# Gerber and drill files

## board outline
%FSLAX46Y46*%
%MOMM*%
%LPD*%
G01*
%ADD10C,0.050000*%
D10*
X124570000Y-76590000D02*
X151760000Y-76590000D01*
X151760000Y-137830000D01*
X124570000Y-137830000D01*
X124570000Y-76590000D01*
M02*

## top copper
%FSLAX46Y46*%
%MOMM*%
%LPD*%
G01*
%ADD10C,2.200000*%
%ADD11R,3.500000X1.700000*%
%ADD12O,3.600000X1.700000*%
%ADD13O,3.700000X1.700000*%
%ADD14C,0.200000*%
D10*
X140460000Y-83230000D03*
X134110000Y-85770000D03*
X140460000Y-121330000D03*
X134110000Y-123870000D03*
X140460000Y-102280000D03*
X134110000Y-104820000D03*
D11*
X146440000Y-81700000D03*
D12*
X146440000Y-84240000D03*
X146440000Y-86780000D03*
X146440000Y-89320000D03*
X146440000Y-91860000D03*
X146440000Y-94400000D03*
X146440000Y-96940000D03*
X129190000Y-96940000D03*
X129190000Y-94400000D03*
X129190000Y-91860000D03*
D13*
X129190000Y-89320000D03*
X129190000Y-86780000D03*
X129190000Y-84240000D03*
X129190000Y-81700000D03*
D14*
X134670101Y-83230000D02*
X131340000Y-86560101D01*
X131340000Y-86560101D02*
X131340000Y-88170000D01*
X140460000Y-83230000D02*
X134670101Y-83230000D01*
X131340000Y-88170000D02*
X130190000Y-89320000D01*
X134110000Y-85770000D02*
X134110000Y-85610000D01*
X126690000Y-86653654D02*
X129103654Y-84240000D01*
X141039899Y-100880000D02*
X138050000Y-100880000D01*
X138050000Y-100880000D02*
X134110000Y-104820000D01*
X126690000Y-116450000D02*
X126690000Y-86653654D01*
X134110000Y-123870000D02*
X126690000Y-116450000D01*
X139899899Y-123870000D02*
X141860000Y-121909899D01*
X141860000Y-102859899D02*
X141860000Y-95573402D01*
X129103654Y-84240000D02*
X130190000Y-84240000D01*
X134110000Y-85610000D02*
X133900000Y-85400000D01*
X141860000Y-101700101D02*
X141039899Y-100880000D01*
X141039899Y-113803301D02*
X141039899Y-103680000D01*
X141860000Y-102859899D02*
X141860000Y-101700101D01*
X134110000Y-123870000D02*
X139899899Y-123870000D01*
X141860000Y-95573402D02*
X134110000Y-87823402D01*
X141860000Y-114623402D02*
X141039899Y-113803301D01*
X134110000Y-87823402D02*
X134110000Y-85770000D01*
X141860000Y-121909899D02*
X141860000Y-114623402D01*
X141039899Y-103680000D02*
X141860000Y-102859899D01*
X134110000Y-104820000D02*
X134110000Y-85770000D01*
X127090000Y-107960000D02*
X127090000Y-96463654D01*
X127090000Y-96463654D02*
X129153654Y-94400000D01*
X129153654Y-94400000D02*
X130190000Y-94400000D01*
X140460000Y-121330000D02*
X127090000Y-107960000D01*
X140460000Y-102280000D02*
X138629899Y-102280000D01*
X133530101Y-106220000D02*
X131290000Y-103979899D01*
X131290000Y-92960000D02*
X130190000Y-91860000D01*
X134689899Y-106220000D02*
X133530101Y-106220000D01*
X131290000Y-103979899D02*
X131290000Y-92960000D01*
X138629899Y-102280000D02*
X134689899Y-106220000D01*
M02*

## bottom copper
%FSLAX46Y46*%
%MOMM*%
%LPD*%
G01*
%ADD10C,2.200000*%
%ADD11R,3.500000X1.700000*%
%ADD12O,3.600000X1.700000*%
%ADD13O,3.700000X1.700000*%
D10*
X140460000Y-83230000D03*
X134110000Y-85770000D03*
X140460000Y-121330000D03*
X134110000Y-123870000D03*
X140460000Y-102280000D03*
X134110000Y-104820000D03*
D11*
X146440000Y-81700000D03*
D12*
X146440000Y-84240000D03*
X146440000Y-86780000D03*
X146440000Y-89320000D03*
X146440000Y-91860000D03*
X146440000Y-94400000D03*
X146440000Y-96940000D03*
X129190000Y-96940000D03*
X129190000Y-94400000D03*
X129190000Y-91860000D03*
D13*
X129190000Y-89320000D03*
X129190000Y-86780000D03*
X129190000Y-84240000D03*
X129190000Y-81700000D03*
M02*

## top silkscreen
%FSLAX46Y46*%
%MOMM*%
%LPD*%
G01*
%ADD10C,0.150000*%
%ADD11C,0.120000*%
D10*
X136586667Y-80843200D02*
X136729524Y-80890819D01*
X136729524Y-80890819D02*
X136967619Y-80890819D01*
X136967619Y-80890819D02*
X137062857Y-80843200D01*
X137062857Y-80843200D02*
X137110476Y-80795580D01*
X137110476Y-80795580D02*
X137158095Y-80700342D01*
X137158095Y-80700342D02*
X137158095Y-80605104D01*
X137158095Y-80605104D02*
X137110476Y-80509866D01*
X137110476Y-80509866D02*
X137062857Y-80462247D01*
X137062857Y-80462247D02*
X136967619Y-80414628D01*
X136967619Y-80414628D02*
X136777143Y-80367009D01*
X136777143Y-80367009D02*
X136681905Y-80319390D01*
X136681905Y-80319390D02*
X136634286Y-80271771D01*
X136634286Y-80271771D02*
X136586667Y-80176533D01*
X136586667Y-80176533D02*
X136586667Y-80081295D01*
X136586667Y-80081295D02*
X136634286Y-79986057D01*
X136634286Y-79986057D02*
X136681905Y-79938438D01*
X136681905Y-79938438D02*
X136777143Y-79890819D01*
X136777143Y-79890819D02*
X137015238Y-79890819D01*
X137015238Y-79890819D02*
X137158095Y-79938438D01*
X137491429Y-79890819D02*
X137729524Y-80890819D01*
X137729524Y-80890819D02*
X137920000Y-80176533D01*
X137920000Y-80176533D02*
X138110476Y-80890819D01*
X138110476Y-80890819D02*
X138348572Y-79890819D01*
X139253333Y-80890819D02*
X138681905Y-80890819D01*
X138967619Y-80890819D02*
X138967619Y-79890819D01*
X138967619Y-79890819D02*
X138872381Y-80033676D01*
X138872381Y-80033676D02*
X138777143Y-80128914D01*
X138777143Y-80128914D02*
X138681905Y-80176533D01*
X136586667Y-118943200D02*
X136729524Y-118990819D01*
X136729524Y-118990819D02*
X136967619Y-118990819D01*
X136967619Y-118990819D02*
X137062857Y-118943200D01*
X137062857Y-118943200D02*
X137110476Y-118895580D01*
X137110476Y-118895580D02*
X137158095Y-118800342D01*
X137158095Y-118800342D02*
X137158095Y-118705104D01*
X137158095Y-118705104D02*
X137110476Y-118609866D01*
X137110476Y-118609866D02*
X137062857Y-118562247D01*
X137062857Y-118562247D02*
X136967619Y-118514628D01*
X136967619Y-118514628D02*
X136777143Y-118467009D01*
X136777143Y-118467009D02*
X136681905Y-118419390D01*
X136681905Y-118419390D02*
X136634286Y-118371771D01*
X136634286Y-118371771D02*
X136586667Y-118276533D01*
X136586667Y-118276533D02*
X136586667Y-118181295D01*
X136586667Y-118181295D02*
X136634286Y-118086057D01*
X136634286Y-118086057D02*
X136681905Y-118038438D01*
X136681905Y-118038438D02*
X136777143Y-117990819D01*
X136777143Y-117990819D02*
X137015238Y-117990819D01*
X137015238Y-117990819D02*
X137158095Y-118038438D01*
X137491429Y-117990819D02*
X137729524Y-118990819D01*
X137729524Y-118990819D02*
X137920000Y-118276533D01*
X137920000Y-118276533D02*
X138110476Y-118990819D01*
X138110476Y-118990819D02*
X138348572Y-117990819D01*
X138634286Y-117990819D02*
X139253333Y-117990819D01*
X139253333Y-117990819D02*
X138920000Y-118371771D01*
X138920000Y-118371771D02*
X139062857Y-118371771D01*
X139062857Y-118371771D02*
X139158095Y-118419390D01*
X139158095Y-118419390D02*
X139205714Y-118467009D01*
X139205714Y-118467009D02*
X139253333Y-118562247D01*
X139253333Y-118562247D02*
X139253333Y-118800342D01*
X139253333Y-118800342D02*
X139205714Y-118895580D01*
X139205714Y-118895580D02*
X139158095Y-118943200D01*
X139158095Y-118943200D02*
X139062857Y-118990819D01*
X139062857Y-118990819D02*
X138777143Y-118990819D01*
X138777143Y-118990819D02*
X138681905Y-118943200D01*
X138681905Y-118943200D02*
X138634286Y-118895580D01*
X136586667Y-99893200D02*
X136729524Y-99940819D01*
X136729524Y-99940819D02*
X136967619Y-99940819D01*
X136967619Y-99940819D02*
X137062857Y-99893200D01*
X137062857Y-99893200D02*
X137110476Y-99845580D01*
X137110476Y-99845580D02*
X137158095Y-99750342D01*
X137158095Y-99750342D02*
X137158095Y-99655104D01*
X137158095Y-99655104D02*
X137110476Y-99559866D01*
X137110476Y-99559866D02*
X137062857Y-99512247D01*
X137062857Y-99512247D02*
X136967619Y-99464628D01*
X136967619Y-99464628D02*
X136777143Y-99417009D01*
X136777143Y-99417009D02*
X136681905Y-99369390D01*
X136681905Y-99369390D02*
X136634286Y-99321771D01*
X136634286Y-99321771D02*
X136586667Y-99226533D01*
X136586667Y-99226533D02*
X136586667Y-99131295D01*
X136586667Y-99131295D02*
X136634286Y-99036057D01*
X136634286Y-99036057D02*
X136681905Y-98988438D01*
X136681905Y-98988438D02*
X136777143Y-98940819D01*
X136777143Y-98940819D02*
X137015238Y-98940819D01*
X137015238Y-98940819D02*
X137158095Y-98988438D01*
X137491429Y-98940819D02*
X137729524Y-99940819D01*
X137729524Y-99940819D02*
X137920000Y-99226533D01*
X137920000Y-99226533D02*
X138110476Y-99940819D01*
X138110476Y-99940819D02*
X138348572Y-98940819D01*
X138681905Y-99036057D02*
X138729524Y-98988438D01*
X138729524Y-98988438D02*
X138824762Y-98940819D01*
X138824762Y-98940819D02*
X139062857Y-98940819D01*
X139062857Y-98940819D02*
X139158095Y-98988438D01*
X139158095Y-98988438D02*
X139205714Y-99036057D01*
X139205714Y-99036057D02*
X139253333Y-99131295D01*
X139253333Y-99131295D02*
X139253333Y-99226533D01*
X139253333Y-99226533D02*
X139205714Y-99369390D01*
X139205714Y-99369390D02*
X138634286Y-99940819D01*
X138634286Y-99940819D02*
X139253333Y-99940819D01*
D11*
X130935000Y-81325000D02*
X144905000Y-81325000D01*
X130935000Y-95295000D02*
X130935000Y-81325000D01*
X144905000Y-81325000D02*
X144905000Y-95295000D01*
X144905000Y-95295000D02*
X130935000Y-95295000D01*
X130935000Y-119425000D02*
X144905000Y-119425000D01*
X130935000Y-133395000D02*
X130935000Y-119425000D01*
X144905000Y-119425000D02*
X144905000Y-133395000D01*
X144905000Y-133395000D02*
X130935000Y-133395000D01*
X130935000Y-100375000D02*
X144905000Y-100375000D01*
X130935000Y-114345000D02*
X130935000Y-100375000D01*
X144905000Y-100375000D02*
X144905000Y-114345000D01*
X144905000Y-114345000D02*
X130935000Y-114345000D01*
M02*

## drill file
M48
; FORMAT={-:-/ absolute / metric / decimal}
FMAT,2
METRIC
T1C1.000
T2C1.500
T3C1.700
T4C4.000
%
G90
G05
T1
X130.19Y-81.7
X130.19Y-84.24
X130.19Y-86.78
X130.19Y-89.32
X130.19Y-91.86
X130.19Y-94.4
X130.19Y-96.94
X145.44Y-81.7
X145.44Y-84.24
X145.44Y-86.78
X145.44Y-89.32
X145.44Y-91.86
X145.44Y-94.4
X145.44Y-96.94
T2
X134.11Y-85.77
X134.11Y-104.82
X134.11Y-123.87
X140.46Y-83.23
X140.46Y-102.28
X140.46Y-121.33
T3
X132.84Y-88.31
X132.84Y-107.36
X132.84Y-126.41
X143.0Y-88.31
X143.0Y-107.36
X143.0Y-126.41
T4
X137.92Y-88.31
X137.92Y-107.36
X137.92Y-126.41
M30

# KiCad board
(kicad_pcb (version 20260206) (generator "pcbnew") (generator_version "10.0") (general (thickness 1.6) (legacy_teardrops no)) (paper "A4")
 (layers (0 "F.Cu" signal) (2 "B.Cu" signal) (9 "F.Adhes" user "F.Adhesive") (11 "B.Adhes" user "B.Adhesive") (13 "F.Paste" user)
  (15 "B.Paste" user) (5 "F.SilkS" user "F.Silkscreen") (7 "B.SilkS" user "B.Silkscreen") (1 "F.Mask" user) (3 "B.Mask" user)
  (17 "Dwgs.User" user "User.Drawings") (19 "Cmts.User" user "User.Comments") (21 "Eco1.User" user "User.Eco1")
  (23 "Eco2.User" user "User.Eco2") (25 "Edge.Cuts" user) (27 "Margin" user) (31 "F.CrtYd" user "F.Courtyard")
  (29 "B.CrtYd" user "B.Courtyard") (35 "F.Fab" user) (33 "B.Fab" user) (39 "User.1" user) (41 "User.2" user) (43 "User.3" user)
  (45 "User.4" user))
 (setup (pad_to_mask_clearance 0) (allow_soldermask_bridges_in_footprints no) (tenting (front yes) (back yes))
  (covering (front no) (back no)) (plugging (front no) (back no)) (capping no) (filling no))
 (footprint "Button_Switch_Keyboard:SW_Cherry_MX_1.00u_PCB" (layer "F.Cu") (at 140.46 83.23)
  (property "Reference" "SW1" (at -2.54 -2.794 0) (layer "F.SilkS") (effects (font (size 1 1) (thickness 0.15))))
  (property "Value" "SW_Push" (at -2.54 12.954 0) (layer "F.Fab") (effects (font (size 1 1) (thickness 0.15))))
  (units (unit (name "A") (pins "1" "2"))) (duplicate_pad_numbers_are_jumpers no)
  (fp_line (start -9.525 -1.905) (end 4.445 -1.905) (stroke (width 0.12) (type solid)) (layer "F.SilkS"))
  (fp_line (start -9.525 12.065) (end -9.525 -1.905) (stroke (width 0.12) (type solid)) (layer "F.SilkS"))
  (fp_line (start 4.445 -1.905) (end 4.445 12.065) (stroke (width 0.12) (type solid)) (layer "F.SilkS"))
  (fp_line (start 4.445 12.065) (end -9.525 12.065) (stroke (width 0.12) (type solid)) (layer "F.SilkS"))
  (pad "" np_thru_hole circle (at -7.62 5.08) (size 1.7 1.7) (drill 1.7) (layers "*.Cu" "*.Mask"))
  (pad "" np_thru_hole circle (at -2.54 5.08) (size 4 4) (drill 4) (layers "*.Cu" "*.Mask"))
  (pad "" np_thru_hole circle (at 2.54 5.08) (size 1.7 1.7) (drill 1.7) (layers "*.Cu" "*.Mask"))
  (pad "1" thru_hole circle (at 0 0) (size 2.2 2.2) (drill 1.5) (layers "*.Cu" "*.Mask") (remove_unused_layers no)
   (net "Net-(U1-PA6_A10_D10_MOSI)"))
  (pad "2" thru_hole circle (at -6.35 2.54) (size 2.2 2.2) (drill 1.5) (layers "*.Cu" "*.Mask") (remove_unused_layers no) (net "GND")))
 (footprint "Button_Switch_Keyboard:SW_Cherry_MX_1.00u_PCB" (layer "F.Cu") (at 140.46 121.33)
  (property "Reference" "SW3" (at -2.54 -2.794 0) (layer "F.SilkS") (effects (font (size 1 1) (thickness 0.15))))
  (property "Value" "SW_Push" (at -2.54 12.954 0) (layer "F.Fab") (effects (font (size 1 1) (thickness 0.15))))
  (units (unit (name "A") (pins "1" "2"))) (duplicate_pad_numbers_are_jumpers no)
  (fp_line (start -9.525 -1.905) (end 4.445 -1.905) (stroke (width 0.12) (type solid)) (layer "F.SilkS"))
  (fp_line (start -9.525 12.065) (end -9.525 -1.905) (stroke (width 0.12) (type solid)) (layer "F.SilkS"))
  (fp_line (start 4.445 -1.905) (end 4.445 12.065) (stroke (width 0.12) (type solid)) (layer "F.SilkS"))
  (fp_line (start 4.445 12.065) (end -9.525 12.065) (stroke (width 0.12) (type solid)) (layer "F.SilkS"))
  (pad "" np_thru_hole circle (at -7.62 5.08) (size 1.7 1.7) (drill 1.7) (layers "*.Cu" "*.Mask"))
  (pad "" np_thru_hole circle (at -2.54 5.08) (size 4 4) (drill 4) (layers "*.Cu" "*.Mask"))
  (pad "" np_thru_hole circle (at 2.54 5.08) (size 1.7 1.7) (drill 1.7) (layers "*.Cu" "*.Mask"))
  (pad "1" thru_hole circle (at 0 0) (size 2.2 2.2) (drill 1.5) (layers "*.Cu" "*.Mask") (remove_unused_layers no)
   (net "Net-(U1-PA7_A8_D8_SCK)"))
  (pad "2" thru_hole circle (at -6.35 2.54) (size 2.2 2.2) (drill 1.5) (layers "*.Cu" "*.Mask") (remove_unused_layers no) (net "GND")))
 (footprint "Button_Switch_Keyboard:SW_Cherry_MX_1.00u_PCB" (layer "F.Cu") (at 140.46 102.28)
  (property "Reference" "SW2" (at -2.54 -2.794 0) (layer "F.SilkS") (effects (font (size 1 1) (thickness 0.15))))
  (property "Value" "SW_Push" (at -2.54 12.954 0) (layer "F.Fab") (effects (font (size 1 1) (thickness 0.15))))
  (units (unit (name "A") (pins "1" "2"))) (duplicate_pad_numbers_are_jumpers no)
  (fp_line (start -9.525 -1.905) (end 4.445 -1.905) (stroke (width 0.12) (type solid)) (layer "F.SilkS"))
  (fp_line (start -9.525 12.065) (end -9.525 -1.905) (stroke (width 0.12) (type solid)) (layer "F.SilkS"))
  (fp_line (start 4.445 -1.905) (end 4.445 12.065) (stroke (width 0.12) (type solid)) (layer "F.SilkS"))
  (fp_line (start 4.445 12.065) (end -9.525 12.065) (stroke (width 0.12) (type solid)) (layer "F.SilkS"))
  (pad "" np_thru_hole circle (at -7.62 5.08) (size 1.7 1.7) (drill 1.7) (layers "*.Cu" "*.Mask"))
  (pad "" np_thru_hole circle (at -2.54 5.08) (size 4 4) (drill 4) (layers "*.Cu" "*.Mask"))
  (pad "" np_thru_hole circle (at 2.54 5.08) (size 1.7 1.7) (drill 1.7) (layers "*.Cu" "*.Mask"))
  (pad "1" thru_hole circle (at 0 0) (size 2.2 2.2) (drill 1.5) (layers "*.Cu" "*.Mask") (remove_unused_layers no)
   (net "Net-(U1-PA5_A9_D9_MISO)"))
  (pad "2" thru_hole circle (at -6.35 2.54) (size 2.2 2.2) (drill 1.5) (layers "*.Cu" "*.Mask") (remove_unused_layers no) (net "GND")))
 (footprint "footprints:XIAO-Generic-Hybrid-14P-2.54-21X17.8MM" (layer "B.Cu") (at 137.815 89.32 180)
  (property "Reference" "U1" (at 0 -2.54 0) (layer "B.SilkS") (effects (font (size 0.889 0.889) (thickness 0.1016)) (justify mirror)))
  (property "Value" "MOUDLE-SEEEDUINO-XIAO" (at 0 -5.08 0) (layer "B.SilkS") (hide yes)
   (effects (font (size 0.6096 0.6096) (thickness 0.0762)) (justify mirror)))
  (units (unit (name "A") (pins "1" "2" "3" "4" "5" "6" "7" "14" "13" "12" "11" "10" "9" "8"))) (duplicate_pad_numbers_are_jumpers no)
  (pad "1" thru_hole rect (at -7.625 7.62 180) (size 3.5 1.7) (drill 1 (offset -1 0)) (layers "*.Cu" "*.Mask") (remove_unused_layers no)
   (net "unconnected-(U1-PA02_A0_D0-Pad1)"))
  (pad "2" thru_hole oval (at -7.625 5.08 180) (size 3.6 1.7) (drill 1 (offset -1 0)) (layers "*.Cu" "*.Mask") (remove_unused_layers no)
   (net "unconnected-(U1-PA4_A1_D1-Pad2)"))
  (pad "3" thru_hole oval (at -7.625 2.54 180) (size 3.6 1.7) (drill 1 (offset -1 0)) (layers "*.Cu" "*.Mask") (remove_unused_layers no)
   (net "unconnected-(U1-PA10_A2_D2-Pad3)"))
  (pad "4" thru_hole oval (at -7.625 0 180) (size 3.6 1.7) (drill 1 (offset -1 0)) (layers "*.Cu" "*.Mask") (remove_unused_layers no)
   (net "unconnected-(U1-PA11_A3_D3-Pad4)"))
  (pad "5" thru_hole oval (at -7.625 -2.54 180) (size 3.6 1.7) (drill 1 (offset -1 0)) (layers "*.Cu" "*.Mask") (remove_unused_layers no)
   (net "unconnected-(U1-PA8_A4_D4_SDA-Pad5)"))
  (pad "6" thru_hole oval (at -7.625 -5.08) (size 3.6 1.7) (drill 1 (offset 1 0)) (layers "*.Cu" "*.Mask") (remove_unused_layers no)
   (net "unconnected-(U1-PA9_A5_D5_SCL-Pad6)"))
  (pad "7" thru_hole oval (at -7.625 -7.62 180) (size 3.6 1.7) (drill 1 (offset -1 0)) (layers "*.Cu" "*.Mask") (remove_unused_layers no)
   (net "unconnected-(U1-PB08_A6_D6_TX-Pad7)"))
  (pad "8" thru_hole oval (at 7.625 -7.62 180) (size 3.6 1.7) (drill 1 (offset 1 0)) (layers "*.Cu" "*.Mask") (remove_unused_layers no)
   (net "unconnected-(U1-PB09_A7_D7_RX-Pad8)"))
  (pad "9" thru_hole oval (at 7.625 -5.08 180) (size 3.6 1.7) (drill 1 (offset 1 0)) (layers "*.Cu" "*.Mask") (remove_unused_layers no)
   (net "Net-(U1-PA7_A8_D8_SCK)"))
  (pad "10" thru_hole oval (at 7.625 -2.54 180) (size 3.6 1.7) (drill 1 (offset 1 0)) (layers "*.Cu" "*.Mask") (remove_unused_layers no)
   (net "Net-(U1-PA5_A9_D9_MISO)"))
  (pad "11" thru_hole oval (at 7.625 0 180) (size 3.7 1.7) (drill 1 (offset 1 0)) (layers "*.Cu" "*.Mask") (remove_unused_layers no)
   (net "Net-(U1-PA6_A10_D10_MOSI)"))
  (pad "12" thru_hole oval (at 7.625 2.54 180) (size 3.7 1.7) (drill 1 (offset 1 0)) (layers "*.Cu" "*.Mask") (remove_unused_layers no)
   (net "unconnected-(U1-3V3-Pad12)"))
  (pad "13" thru_hole oval (at 7.625 5.08 180) (size 3.7 1.7) (drill 1 (offset 1 0)) (layers "*.Cu" "*.Mask") (remove_unused_layers no)
   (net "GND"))
  (pad "14" thru_hole oval (at 7.625 7.62 180) (size 3.7 1.7) (drill 1 (offset 1 0)) (layers "*.Cu" "*.Mask") (remove_unused_layers no)
   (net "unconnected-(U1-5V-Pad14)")))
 (gr_rect (start 124.57 76.59) (end 151.76 137.83) (stroke (width 0.05) (type default)) (fill no) (layer "Edge.Cuts"))
 (segment (start 134.670101 83.23) (end 131.34 86.560101) (width 0.2) (layer "F.Cu") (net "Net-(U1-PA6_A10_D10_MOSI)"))
 (segment (start 131.34 86.560101) (end 131.34 88.17) (width 0.2) (layer "F.Cu") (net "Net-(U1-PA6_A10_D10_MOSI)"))
 (segment (start 140.46 83.23) (end 134.670101 83.23) (width 0.2) (layer "F.Cu") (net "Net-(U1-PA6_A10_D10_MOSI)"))
 (segment (start 131.34 88.17) (end 130.19 89.32) (width 0.2) (layer "F.Cu") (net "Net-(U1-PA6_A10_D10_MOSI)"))
 (segment (start 134.11 85.77) (end 134.11 85.61) (width 0.2) (layer "F.Cu") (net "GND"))
 (segment (start 126.69 86.653654) (end 129.103654 84.24) (width 0.2) (layer "F.Cu") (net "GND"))
 (segment (start 141.039899 100.88) (end 138.05 100.88) (width 0.2) (layer "F.Cu") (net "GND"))
 (segment (start 138.05 100.88) (end 134.11 104.82) (width 0.2) (layer "F.Cu") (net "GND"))
 (segment (start 126.69 116.45) (end 126.69 86.653654) (width 0.2) (layer "F.Cu") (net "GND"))
 (segment (start 134.11 123.87) (end 126.69 116.45) (width 0.2) (layer "F.Cu") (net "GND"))
 (segment (start 139.899899 123.87) (end 141.86 121.909899) (width 0.2) (layer "F.Cu") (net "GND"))
 (segment (start 141.86 102.859899) (end 141.86 95.573402) (width 0.2) (layer "F.Cu") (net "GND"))
 (segment (start 129.103654 84.24) (end 130.19 84.24) (width 0.2) (layer "F.Cu") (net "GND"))
 (segment (start 134.11 85.61) (end 133.9 85.4) (width 0.2) (layer "F.Cu") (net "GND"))
 (segment (start 141.86 101.700101) (end 141.039899 100.88) (width 0.2) (layer "F.Cu") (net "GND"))
 (segment (start 141.039899 113.803301) (end 141.039899 103.68) (width 0.2) (layer "F.Cu") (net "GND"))
 (segment (start 141.86 102.859899) (end 141.86 101.700101) (width 0.2) (layer "F.Cu") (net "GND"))
 (segment (start 134.11 123.87) (end 139.899899 123.87) (width 0.2) (layer "F.Cu") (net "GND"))
 (segment (start 141.86 95.573402) (end 134.11 87.823402) (width 0.2) (layer "F.Cu") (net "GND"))
 (segment (start 141.86 114.623402) (end 141.039899 113.803301) (width 0.2) (layer "F.Cu") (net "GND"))
 (segment (start 134.11 87.823402) (end 134.11 85.77) (width 0.2) (layer "F.Cu") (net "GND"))
 (segment (start 141.86 121.909899) (end 141.86 114.623402) (width 0.2) (layer "F.Cu") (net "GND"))
 (segment (start 141.039899 103.68) (end 141.86 102.859899) (width 0.2) (layer "F.Cu") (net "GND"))
 (segment (start 134.11 104.82) (end 134.11 85.77) (width 0.2) (layer "F.Cu") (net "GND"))
 (segment (start 127.09 107.96) (end 127.09 96.463654) (width 0.2) (layer "F.Cu") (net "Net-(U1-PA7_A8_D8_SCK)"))
 (segment (start 127.09 96.463654) (end 129.153654 94.4) (width 0.2) (layer "F.Cu") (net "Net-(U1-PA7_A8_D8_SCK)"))
 (segment (start 129.153654 94.4) (end 130.19 94.4) (width 0.2) (layer "F.Cu") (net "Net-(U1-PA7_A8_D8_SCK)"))
 (segment (start 140.46 121.33) (end 127.09 107.96) (width 0.2) (layer "F.Cu") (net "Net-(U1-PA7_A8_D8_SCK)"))
 (segment (start 140.46 102.28) (end 138.629899 102.28) (width 0.2) (layer "F.Cu") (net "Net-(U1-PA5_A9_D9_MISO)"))
 (segment (start 133.530101 106.22) (end 131.29 103.979899) (width 0.2) (layer "F.Cu") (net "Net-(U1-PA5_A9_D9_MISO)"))
 (segment (start 131.29 92.96) (end 130.19 91.86) (width 0.2) (layer "F.Cu") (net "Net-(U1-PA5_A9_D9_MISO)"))
 (segment (start 134.689899 106.22) (end 133.530101 106.22) (width 0.2) (layer "F.Cu") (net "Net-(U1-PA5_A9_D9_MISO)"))
 (segment (start 131.29 103.979899) (end 131.29 92.96) (width 0.2) (layer "F.Cu") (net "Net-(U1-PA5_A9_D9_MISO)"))
 (segment (start 138.629899 102.28) (end 134.689899 106.22) (width 0.2) (layer "F.Cu") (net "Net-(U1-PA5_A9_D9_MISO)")))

